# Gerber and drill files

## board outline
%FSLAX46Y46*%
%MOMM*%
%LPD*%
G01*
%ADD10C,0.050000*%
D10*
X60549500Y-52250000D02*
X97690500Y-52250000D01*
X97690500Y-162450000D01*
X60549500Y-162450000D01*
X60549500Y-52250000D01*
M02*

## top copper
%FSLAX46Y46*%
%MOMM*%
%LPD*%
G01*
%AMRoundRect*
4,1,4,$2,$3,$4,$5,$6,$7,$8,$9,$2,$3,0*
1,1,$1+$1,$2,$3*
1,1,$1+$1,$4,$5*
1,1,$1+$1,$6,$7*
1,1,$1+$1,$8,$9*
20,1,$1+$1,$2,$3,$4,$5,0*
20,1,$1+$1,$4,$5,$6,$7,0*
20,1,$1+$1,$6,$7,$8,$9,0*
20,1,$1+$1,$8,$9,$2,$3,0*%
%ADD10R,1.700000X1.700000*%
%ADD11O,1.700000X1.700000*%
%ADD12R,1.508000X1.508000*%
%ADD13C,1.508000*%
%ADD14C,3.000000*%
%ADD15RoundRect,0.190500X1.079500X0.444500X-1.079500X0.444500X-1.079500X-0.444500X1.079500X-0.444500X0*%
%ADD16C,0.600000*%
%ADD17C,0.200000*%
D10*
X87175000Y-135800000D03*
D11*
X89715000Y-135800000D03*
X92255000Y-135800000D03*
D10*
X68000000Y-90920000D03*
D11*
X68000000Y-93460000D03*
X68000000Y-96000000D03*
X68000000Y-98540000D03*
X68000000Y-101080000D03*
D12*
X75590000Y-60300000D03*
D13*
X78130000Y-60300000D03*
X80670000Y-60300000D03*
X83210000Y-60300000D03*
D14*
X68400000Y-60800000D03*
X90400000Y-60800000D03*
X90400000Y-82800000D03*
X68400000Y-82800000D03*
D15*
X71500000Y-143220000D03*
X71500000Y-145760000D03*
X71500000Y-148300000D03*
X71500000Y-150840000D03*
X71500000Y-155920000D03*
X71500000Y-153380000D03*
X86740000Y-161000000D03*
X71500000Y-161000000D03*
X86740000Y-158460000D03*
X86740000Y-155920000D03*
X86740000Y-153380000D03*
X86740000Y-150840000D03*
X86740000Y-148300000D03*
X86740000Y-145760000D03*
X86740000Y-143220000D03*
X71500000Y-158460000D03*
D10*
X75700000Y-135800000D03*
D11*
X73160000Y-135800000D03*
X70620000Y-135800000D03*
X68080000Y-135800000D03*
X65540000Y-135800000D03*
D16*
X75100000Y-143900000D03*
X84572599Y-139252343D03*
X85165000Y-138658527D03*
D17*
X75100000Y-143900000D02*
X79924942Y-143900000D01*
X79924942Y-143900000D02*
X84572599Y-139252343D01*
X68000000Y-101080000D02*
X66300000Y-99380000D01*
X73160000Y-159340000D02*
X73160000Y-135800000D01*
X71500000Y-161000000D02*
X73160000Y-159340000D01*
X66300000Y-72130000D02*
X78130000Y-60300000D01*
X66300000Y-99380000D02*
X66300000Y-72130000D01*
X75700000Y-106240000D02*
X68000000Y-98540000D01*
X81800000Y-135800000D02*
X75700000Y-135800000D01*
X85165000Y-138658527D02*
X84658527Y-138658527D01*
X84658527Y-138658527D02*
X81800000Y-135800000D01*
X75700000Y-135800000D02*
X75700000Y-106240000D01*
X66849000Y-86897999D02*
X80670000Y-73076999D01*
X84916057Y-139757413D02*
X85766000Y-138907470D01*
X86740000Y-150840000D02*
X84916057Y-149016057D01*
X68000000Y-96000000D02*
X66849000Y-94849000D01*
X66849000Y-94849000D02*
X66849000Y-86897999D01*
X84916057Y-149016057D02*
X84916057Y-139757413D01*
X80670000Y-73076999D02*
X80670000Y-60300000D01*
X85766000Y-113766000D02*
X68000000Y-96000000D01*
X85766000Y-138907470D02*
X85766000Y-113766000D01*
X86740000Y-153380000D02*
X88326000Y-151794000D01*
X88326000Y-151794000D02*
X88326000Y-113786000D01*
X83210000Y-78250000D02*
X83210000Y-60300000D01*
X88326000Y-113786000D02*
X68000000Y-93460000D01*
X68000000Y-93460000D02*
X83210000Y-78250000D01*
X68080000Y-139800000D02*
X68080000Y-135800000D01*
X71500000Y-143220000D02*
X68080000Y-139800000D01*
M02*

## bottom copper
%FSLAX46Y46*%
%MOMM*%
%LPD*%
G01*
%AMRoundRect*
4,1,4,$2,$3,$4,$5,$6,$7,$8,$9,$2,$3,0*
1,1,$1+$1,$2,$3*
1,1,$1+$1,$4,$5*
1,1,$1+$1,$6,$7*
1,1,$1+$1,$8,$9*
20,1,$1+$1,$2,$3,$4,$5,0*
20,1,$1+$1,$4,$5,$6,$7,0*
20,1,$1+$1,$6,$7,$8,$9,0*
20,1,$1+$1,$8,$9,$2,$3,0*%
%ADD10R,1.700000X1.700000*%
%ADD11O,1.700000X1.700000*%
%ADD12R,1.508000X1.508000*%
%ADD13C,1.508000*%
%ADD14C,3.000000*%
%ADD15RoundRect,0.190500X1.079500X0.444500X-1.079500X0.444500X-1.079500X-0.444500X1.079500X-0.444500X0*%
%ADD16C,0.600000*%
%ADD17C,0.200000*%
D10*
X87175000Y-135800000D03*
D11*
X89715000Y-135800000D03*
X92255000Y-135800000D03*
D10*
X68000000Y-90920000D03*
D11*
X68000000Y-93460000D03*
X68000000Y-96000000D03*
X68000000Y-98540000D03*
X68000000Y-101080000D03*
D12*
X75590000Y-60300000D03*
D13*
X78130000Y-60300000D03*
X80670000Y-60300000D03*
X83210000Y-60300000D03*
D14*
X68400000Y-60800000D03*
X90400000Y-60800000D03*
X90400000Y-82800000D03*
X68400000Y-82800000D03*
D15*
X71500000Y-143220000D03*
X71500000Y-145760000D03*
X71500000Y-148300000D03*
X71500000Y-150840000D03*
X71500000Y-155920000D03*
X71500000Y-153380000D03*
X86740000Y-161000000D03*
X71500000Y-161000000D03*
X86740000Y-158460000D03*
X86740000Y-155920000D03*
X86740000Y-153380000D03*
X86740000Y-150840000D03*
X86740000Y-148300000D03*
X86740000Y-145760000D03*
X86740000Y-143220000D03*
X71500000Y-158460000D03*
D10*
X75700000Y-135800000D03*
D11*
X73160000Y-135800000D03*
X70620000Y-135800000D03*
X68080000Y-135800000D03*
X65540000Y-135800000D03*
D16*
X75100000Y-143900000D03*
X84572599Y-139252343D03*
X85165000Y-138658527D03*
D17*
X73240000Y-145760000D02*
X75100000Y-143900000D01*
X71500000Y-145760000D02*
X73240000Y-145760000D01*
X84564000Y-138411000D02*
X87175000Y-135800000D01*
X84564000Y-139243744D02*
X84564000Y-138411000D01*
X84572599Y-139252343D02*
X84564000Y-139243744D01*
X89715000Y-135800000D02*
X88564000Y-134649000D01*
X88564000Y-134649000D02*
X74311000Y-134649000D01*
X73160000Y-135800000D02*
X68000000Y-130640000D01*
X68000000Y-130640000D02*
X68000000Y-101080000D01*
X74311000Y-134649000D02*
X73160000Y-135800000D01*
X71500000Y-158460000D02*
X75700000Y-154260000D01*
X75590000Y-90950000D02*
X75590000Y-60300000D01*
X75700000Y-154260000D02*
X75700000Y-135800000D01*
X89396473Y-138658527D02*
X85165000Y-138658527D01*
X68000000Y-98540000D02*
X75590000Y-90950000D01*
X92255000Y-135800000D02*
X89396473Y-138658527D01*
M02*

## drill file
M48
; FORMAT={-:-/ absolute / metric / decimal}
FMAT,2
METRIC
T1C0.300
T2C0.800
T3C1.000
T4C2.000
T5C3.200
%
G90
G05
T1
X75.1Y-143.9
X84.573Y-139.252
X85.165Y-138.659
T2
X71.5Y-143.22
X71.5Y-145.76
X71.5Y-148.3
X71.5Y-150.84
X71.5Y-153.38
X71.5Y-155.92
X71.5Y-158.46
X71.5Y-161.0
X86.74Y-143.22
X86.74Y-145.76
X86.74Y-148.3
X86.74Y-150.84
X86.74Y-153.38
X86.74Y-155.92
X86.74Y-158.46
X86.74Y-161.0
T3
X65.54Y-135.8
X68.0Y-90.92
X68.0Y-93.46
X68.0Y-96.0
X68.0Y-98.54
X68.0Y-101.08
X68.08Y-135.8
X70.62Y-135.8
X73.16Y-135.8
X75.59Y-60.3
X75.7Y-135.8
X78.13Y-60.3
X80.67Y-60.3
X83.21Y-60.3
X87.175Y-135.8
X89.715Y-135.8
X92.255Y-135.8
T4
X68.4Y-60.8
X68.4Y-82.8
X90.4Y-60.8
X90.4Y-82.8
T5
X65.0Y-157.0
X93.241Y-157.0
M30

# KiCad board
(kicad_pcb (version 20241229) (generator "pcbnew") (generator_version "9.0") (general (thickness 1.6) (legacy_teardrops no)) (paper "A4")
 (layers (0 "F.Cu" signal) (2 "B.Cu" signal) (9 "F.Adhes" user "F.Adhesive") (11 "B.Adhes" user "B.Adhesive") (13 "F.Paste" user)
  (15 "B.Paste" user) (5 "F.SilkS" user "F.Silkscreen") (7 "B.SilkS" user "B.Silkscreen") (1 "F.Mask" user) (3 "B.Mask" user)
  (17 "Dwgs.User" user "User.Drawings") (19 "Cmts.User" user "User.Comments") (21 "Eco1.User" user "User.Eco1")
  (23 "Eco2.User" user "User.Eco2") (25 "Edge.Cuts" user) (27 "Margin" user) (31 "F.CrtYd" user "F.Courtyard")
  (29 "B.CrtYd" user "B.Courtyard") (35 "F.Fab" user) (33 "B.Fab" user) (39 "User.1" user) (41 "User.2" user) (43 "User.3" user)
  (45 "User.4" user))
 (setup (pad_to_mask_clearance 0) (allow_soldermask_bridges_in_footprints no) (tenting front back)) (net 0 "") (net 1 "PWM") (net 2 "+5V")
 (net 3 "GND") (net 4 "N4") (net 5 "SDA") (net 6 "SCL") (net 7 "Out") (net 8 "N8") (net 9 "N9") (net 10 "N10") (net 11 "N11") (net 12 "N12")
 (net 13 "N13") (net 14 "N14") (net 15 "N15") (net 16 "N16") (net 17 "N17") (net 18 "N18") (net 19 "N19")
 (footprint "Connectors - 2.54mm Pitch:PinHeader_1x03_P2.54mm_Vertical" (layer "F.Cu") (at 87.175 135.8 90)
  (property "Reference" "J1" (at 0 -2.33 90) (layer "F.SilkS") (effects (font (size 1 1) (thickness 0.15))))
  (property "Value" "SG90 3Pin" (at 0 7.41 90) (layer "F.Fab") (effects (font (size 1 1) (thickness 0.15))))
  (pad "1" thru_hole rect (at 0 0 90) (size 1.7 1.7) (drill 1) (layers "*.Cu" "*.Mask") (remove_unused_layers no) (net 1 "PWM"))
  (pad "2" thru_hole oval (at 0 2.54 90) (size 1.7 1.7) (drill 1) (layers "*.Cu" "*.Mask") (remove_unused_layers no) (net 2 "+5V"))
  (pad "3" thru_hole oval (at 0 5.08 90) (size 1.7 1.7) (drill 1) (layers "*.Cu" "*.Mask") (remove_unused_layers no) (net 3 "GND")))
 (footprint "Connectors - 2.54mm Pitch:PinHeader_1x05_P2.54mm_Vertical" (layer "F.Cu") (at 68 90.92)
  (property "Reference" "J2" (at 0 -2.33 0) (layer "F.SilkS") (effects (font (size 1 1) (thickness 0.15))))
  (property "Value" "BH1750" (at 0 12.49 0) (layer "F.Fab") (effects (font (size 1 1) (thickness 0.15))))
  (pad "1" thru_hole rect (at 0 0) (size 1.7 1.7) (drill 1) (layers "*.Cu" "*.Mask") (remove_unused_layers no) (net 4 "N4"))
  (pad "2" thru_hole oval (at 0 2.54) (size 1.7 1.7) (drill 1) (layers "*.Cu" "*.Mask") (remove_unused_layers no) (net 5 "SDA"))
  (pad "3" thru_hole oval (at 0 5.08) (size 1.7 1.7) (drill 1) (layers "*.Cu" "*.Mask") (remove_unused_layers no) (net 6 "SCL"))
  (pad "4" thru_hole oval (at 0 7.62) (size 1.7 1.7) (drill 1) (layers "*.Cu" "*.Mask") (remove_unused_layers no) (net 3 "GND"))
  (pad "5" thru_hole oval (at 0 10.16) (size 1.7 1.7) (drill 1) (layers "*.Cu" "*.Mask") (remove_unused_layers no) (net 2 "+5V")))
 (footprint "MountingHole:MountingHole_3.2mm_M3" (layer "F.Cu") (at 65 157)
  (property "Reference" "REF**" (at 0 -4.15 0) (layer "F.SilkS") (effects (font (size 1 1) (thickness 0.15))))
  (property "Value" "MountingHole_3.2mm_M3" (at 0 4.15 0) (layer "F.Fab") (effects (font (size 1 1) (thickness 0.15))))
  (pad "" np_thru_hole circle (at 0 0) (size 3.2 3.2) (drill 3.2) (layers "*.Cu" "*.Mask")))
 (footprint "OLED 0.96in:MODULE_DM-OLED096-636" (layer "F.Cu") (at 79.4 71.8)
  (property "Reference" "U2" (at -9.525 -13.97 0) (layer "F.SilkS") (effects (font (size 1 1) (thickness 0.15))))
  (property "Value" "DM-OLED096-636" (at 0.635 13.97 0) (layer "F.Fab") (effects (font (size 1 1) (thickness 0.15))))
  (pad "1" thru_hole rect (at -3.81 -11.5) (size 1.508 1.508) (drill 1) (layers "*.Cu" "*.Mask") (remove_unused_layers no) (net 3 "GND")
   (solder_mask_margin 0.102))
  (pad "2" thru_hole circle (at -1.27 -11.5) (size 1.508 1.508) (drill 1) (layers "*.Cu" "*.Mask") (remove_unused_layers no) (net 2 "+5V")
   (solder_mask_margin 0.102))
  (pad "3" thru_hole circle (at 1.27 -11.5) (size 1.508 1.508) (drill 1) (layers "*.Cu" "*.Mask") (remove_unused_layers no) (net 6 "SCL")
   (solder_mask_margin 0.102))
  (pad "4" thru_hole circle (at 3.81 -11.5) (size 1.508 1.508) (drill 1) (layers "*.Cu" "*.Mask") (remove_unused_layers no) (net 5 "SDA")
   (solder_mask_margin 0.102))
  (pad "S1" thru_hole circle (at -11 -11) (size 3 3) (drill 2) (layers "*.Cu" "*.Mask") (remove_unused_layers no) (solder_mask_margin 0.102))
  (pad "S2" thru_hole circle (at 11 -11) (size 3 3) (drill 2) (layers "*.Cu" "*.Mask") (remove_unused_layers no) (solder_mask_margin 0.102))
  (pad "S3" thru_hole circle (at 11 11) (size 3 3) (drill 2) (layers "*.Cu" "*.Mask") (remove_unused_layers no) (solder_mask_margin 0.102))
  (pad "S4" thru_hole circle (at -11 11) (size 3 3) (drill 2) (layers "*.Cu" "*.Mask") (remove_unused_layers no) (solder_mask_margin 0.102)))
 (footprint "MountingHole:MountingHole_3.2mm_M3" (layer "F.Cu") (at 93.241 157)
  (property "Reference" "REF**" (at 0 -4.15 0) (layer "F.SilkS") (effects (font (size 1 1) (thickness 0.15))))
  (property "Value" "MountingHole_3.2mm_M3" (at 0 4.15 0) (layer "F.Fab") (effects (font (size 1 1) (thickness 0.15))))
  (pad "" np_thru_hole circle (at 0 0) (size 3.2 3.2) (drill 3.2) (layers "*.Cu" "*.Mask")))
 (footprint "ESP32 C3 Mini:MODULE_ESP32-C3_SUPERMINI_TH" (layer "F.Cu") (at 79.12 151.1 180)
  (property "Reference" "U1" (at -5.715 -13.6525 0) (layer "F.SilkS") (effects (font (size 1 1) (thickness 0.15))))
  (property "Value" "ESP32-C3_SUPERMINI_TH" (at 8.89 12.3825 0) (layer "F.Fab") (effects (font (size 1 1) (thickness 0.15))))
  (pad "0" thru_hole roundrect (at 7.62 7.88 180) (size 2.54 1.27) (drill 0.8) (layers "*.Cu" "*.Mask") (remove_unused_layers no)
   (roundrect_rratio 0.15) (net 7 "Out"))
  (pad "1" thru_hole roundrect (at 7.62 5.34 180) (size 2.54 1.27) (drill 0.8) (layers "*.Cu" "*.Mask") (remove_unused_layers no)
   (roundrect_rratio 0.15) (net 1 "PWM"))
  (pad "2" thru_hole roundrect (at 7.62 2.8 180) (size 2.54 1.27) (drill 0.8) (layers "*.Cu" "*.Mask") (remove_unused_layers no)
   (roundrect_rratio 0.15) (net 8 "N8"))
  (pad "3" thru_hole roundrect (at 7.62 0.26 180) (size 2.54 1.27) (drill 0.8) (layers "*.Cu" "*.Mask") (remove_unused_layers no)
   (roundrect_rratio 0.15) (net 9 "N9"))
  (pad "3.3" thru_hole roundrect (at 7.62 -4.82 180) (size 2.54 1.27) (drill 0.8) (layers "*.Cu" "*.Mask") (remove_unused_layers no)
   (roundrect_rratio 0.15) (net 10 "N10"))
  (pad "4" thru_hole roundrect (at 7.62 -2.28 180) (size 2.54 1.27) (drill 0.8) (layers "*.Cu" "*.Mask") (remove_unused_layers no)
   (roundrect_rratio 0.15) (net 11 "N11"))
  (pad "5" thru_hole roundrect (at -7.62 -9.9 180) (size 2.54 1.27) (drill 0.8) (layers "*.Cu" "*.Mask") (remove_unused_layers no)
   (roundrect_rratio 0.15) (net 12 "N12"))
  (pad "5V" thru_hole roundrect (at 7.62 -9.9 180) (size 2.54 1.27) (drill 0.8) (layers "*.Cu" "*.Mask") (remove_unused_layers no)
   (roundrect_rratio 0.15) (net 2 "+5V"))
  (pad "6" thru_hole roundrect (at -7.62 -7.36 180) (size 2.54 1.27) (drill 0.8) (layers "*.Cu" "*.Mask") (remove_unused_layers no)
   (roundrect_rratio 0.15) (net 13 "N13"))
  (pad "7" thru_hole roundrect (at -7.62 -4.82 180) (size 2.54 1.27) (drill 0.8) (layers "*.Cu" "*.Mask") (remove_unused_layers no)
   (roundrect_rratio 0.15) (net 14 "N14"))
  (pad "8" thru_hole roundrect (at -7.62 -2.28 180) (size 2.54 1.27) (drill 0.8) (layers "*.Cu" "*.Mask") (remove_unused_layers no)
   (roundrect_rratio 0.15) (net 5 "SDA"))
  (pad "9" thru_hole roundrect (at -7.62 0.26 180) (size 2.54 1.27) (drill 0.8) (layers "*.Cu" "*.Mask") (remove_unused_layers no)
   (roundrect_rratio 0.15) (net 6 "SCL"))
  (pad "10" thru_hole roundrect (at -7.62 2.8 180) (size 2.54 1.27) (drill 0.8) (layers "*.Cu" "*.Mask") (remove_unused_layers no)
   (roundrect_rratio 0.15) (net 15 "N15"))
  (pad "20" thru_hole roundrect (at -7.62 5.34 180) (size 2.54 1.27) (drill 0.8) (layers "*.Cu" "*.Mask") (remove_unused_layers no)
   (roundrect_rratio 0.15) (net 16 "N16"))
  (pad "21" thru_hole roundrect (at -7.62 7.88 180) (size 2.54 1.27) (drill 0.8) (layers "*.Cu" "*.Mask") (remove_unused_layers no)
   (roundrect_rratio 0.15) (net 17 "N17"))
  (pad "G" thru_hole roundrect (at 7.62 -7.36 180) (size 2.54 1.27) (drill 0.8) (layers "*.Cu" "*.Mask" "B.SilkS") (remove_unused_layers no)
   (roundrect_rratio 0.15) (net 3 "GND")))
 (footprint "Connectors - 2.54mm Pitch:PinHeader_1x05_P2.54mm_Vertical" (layer "F.Cu") (at 75.7 135.8 -90)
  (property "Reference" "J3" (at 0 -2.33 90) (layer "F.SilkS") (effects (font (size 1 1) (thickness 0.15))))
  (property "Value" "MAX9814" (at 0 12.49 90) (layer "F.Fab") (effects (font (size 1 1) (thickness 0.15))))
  (pad "1" thru_hole rect (at 0 0 270) (size 1.7 1.7) (drill 1) (layers "*.Cu" "*.Mask") (remove_unused_layers no) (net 3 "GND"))
  (pad "2" thru_hole oval (at 0 2.54 270) (size 1.7 1.7) (drill 1) (layers "*.Cu" "*.Mask") (remove_unused_layers no) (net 2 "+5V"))
  (pad "3" thru_hole oval (at 0 5.08 270) (size 1.7 1.7) (drill 1) (layers "*.Cu" "*.Mask") (remove_unused_layers no) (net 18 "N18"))
  (pad "4" thru_hole oval (at 0 7.62 270) (size 1.7 1.7) (drill 1) (layers "*.Cu" "*.Mask") (remove_unused_layers no) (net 7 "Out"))
  (pad "5" thru_hole oval (at 0 10.16 270) (size 1.7 1.7) (drill 1) (layers "*.Cu" "*.Mask") (remove_unused_layers no) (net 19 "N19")))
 (gr_rect (start 60.5495 52.25) (end 97.6905 162.45) (stroke (width 0.05) (type solid)) (fill no) (layer "Edge.Cuts"))
 (segment (start 75.1 143.9) (end 79.924942 143.9) (width 0.2) (layer "F.Cu") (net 1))
 (segment (start 79.924942 143.9) (end 84.572599 139.252343) (width 0.2) (layer "F.Cu") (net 1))
 (via (at 75.1 143.9) (size 0.6) (drill 0.3) (layers "F.Cu" "B.Cu") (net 1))
 (via (at 84.572599 139.252343) (size 0.6) (drill 0.3) (layers "F.Cu" "B.Cu") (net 1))
 (segment (start 73.24 145.76) (end 75.1 143.9) (width 0.2) (layer "B.Cu") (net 1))
 (segment (start 71.5 145.76) (end 73.24 145.76) (width 0.2) (layer "B.Cu") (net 1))
 (segment (start 84.564 138.411) (end 87.175 135.8) (width 0.2) (layer "B.Cu") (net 1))
 (segment (start 84.564 139.243744) (end 84.564 138.411) (width 0.2) (layer "B.Cu") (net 1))
 (segment (start 84.572599 139.252343) (end 84.564 139.243744) (width 0.2) (layer "B.Cu") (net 1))
 (segment (start 68 101.08) (end 66.3 99.38) (width 0.2) (layer "F.Cu") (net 2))
 (segment (start 73.16 159.34) (end 73.16 135.8) (width 0.2) (layer "F.Cu") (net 2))
 (segment (start 71.5 161) (end 73.16 159.34) (width 0.2) (layer "F.Cu") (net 2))
 (segment (start 66.3 72.13) (end 78.13 60.3) (width 0.2) (layer "F.Cu") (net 2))
 (segment (start 66.3 99.38) (end 66.3 72.13) (width 0.2) (layer "F.Cu") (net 2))
 (segment (start 89.715 135.8) (end 88.564 134.649) (width 0.2) (layer "B.Cu") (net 2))
 (segment (start 88.564 134.649) (end 74.311 134.649) (width 0.2) (layer "B.Cu") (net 2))
 (segment (start 73.16 135.8) (end 68 130.64) (width 0.2) (layer "B.Cu") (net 2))
 (segment (start 68 130.64) (end 68 101.08) (width 0.2) (layer "B.Cu") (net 2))
 (segment (start 74.311 134.649) (end 73.16 135.8) (width 0.2) (layer "B.Cu") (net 2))
 (segment (start 75.7 106.24) (end 68 98.54) (width 0.2) (layer "F.Cu") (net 3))
 (segment (start 81.8 135.8) (end 75.7 135.8) (width 0.2) (layer "F.Cu") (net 3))
 (segment (start 85.165 138.658527) (end 84.658527 138.658527) (width 0.2) (layer "F.Cu") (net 3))
 (segment (start 84.658527 138.658527) (end 81.8 135.8) (width 0.2) (layer "F.Cu") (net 3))
 (segment (start 75.7 135.8) (end 75.7 106.24) (width 0.2) (layer "F.Cu") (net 3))
 (via (at 85.165 138.658527) (size 0.6) (drill 0.3) (layers "F.Cu" "B.Cu") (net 3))
 (segment (start 71.5 158.46) (end 75.7 154.26) (width 0.2) (layer "B.Cu") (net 3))
 (segment (start 75.59 90.95) (end 75.59 60.3) (width 0.2) (layer "B.Cu") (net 3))
 (segment (start 75.7 154.26) (end 75.7 135.8) (width 0.2) (layer "B.Cu") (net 3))
 (segment (start 89.396473 138.658527) (end 85.165 138.658527) (width 0.2) (layer "B.Cu") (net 3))
 (segment (start 68 98.54) (end 75.59 90.95) (width 0.2) (layer "B.Cu") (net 3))
 (segment (start 92.255 135.8) (end 89.396473 138.658527) (width 0.2) (layer "B.Cu") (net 3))
 (segment (start 66.849 86.897999) (end 80.67 73.076999) (width 0.2) (layer "F.Cu") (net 6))
 (segment (start 84.916057 139.757413) (end 85.766 138.90747) (width 0.2) (layer "F.Cu") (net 6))
 (segment (start 86.74 150.84) (end 84.916057 149.016057) (width 0.2) (layer "F.Cu") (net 6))
 (segment (start 68 96) (end 66.849 94.849) (width 0.2) (layer "F.Cu") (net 6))
 (segment (start 66.849 94.849) (end 66.849 86.897999) (width 0.2) (layer "F.Cu") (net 6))
 (segment (start 84.916057 149.016057) (end 84.916057 139.757413) (width 0.2) (layer "F.Cu") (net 6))
 (segment (start 80.67 73.076999) (end 80.67 60.3) (width 0.2) (layer "F.Cu") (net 6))
 (segment (start 85.766 113.766) (end 68 96) (width 0.2) (layer "F.Cu") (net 6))
 (segment (start 85.766 138.90747) (end 85.766 113.766) (width 0.2) (layer "F.Cu") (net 6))
 (segment (start 86.74 153.38) (end 88.326 151.794) (width 0.2) (layer "F.Cu") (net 5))
 (segment (start 88.326 151.794) (end 88.326 113.786) (width 0.2) (layer "F.Cu") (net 5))
 (segment (start 83.21 78.25) (end 83.21 60.3) (width 0.2) (layer "F.Cu") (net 5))
 (segment (start 88.326 113.786) (end 68 93.46) (width 0.2) (layer "F.Cu") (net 5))
 (segment (start 68 93.46) (end 83.21 78.25) (width 0.2) (layer "F.Cu") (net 5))
 (segment (start 68.08 139.8) (end 68.08 135.8) (width 0.2) (layer "F.Cu") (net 7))
 (segment (start 71.5 143.22) (end 68.08 139.8) (width 0.2) (layer "F.Cu") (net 7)))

